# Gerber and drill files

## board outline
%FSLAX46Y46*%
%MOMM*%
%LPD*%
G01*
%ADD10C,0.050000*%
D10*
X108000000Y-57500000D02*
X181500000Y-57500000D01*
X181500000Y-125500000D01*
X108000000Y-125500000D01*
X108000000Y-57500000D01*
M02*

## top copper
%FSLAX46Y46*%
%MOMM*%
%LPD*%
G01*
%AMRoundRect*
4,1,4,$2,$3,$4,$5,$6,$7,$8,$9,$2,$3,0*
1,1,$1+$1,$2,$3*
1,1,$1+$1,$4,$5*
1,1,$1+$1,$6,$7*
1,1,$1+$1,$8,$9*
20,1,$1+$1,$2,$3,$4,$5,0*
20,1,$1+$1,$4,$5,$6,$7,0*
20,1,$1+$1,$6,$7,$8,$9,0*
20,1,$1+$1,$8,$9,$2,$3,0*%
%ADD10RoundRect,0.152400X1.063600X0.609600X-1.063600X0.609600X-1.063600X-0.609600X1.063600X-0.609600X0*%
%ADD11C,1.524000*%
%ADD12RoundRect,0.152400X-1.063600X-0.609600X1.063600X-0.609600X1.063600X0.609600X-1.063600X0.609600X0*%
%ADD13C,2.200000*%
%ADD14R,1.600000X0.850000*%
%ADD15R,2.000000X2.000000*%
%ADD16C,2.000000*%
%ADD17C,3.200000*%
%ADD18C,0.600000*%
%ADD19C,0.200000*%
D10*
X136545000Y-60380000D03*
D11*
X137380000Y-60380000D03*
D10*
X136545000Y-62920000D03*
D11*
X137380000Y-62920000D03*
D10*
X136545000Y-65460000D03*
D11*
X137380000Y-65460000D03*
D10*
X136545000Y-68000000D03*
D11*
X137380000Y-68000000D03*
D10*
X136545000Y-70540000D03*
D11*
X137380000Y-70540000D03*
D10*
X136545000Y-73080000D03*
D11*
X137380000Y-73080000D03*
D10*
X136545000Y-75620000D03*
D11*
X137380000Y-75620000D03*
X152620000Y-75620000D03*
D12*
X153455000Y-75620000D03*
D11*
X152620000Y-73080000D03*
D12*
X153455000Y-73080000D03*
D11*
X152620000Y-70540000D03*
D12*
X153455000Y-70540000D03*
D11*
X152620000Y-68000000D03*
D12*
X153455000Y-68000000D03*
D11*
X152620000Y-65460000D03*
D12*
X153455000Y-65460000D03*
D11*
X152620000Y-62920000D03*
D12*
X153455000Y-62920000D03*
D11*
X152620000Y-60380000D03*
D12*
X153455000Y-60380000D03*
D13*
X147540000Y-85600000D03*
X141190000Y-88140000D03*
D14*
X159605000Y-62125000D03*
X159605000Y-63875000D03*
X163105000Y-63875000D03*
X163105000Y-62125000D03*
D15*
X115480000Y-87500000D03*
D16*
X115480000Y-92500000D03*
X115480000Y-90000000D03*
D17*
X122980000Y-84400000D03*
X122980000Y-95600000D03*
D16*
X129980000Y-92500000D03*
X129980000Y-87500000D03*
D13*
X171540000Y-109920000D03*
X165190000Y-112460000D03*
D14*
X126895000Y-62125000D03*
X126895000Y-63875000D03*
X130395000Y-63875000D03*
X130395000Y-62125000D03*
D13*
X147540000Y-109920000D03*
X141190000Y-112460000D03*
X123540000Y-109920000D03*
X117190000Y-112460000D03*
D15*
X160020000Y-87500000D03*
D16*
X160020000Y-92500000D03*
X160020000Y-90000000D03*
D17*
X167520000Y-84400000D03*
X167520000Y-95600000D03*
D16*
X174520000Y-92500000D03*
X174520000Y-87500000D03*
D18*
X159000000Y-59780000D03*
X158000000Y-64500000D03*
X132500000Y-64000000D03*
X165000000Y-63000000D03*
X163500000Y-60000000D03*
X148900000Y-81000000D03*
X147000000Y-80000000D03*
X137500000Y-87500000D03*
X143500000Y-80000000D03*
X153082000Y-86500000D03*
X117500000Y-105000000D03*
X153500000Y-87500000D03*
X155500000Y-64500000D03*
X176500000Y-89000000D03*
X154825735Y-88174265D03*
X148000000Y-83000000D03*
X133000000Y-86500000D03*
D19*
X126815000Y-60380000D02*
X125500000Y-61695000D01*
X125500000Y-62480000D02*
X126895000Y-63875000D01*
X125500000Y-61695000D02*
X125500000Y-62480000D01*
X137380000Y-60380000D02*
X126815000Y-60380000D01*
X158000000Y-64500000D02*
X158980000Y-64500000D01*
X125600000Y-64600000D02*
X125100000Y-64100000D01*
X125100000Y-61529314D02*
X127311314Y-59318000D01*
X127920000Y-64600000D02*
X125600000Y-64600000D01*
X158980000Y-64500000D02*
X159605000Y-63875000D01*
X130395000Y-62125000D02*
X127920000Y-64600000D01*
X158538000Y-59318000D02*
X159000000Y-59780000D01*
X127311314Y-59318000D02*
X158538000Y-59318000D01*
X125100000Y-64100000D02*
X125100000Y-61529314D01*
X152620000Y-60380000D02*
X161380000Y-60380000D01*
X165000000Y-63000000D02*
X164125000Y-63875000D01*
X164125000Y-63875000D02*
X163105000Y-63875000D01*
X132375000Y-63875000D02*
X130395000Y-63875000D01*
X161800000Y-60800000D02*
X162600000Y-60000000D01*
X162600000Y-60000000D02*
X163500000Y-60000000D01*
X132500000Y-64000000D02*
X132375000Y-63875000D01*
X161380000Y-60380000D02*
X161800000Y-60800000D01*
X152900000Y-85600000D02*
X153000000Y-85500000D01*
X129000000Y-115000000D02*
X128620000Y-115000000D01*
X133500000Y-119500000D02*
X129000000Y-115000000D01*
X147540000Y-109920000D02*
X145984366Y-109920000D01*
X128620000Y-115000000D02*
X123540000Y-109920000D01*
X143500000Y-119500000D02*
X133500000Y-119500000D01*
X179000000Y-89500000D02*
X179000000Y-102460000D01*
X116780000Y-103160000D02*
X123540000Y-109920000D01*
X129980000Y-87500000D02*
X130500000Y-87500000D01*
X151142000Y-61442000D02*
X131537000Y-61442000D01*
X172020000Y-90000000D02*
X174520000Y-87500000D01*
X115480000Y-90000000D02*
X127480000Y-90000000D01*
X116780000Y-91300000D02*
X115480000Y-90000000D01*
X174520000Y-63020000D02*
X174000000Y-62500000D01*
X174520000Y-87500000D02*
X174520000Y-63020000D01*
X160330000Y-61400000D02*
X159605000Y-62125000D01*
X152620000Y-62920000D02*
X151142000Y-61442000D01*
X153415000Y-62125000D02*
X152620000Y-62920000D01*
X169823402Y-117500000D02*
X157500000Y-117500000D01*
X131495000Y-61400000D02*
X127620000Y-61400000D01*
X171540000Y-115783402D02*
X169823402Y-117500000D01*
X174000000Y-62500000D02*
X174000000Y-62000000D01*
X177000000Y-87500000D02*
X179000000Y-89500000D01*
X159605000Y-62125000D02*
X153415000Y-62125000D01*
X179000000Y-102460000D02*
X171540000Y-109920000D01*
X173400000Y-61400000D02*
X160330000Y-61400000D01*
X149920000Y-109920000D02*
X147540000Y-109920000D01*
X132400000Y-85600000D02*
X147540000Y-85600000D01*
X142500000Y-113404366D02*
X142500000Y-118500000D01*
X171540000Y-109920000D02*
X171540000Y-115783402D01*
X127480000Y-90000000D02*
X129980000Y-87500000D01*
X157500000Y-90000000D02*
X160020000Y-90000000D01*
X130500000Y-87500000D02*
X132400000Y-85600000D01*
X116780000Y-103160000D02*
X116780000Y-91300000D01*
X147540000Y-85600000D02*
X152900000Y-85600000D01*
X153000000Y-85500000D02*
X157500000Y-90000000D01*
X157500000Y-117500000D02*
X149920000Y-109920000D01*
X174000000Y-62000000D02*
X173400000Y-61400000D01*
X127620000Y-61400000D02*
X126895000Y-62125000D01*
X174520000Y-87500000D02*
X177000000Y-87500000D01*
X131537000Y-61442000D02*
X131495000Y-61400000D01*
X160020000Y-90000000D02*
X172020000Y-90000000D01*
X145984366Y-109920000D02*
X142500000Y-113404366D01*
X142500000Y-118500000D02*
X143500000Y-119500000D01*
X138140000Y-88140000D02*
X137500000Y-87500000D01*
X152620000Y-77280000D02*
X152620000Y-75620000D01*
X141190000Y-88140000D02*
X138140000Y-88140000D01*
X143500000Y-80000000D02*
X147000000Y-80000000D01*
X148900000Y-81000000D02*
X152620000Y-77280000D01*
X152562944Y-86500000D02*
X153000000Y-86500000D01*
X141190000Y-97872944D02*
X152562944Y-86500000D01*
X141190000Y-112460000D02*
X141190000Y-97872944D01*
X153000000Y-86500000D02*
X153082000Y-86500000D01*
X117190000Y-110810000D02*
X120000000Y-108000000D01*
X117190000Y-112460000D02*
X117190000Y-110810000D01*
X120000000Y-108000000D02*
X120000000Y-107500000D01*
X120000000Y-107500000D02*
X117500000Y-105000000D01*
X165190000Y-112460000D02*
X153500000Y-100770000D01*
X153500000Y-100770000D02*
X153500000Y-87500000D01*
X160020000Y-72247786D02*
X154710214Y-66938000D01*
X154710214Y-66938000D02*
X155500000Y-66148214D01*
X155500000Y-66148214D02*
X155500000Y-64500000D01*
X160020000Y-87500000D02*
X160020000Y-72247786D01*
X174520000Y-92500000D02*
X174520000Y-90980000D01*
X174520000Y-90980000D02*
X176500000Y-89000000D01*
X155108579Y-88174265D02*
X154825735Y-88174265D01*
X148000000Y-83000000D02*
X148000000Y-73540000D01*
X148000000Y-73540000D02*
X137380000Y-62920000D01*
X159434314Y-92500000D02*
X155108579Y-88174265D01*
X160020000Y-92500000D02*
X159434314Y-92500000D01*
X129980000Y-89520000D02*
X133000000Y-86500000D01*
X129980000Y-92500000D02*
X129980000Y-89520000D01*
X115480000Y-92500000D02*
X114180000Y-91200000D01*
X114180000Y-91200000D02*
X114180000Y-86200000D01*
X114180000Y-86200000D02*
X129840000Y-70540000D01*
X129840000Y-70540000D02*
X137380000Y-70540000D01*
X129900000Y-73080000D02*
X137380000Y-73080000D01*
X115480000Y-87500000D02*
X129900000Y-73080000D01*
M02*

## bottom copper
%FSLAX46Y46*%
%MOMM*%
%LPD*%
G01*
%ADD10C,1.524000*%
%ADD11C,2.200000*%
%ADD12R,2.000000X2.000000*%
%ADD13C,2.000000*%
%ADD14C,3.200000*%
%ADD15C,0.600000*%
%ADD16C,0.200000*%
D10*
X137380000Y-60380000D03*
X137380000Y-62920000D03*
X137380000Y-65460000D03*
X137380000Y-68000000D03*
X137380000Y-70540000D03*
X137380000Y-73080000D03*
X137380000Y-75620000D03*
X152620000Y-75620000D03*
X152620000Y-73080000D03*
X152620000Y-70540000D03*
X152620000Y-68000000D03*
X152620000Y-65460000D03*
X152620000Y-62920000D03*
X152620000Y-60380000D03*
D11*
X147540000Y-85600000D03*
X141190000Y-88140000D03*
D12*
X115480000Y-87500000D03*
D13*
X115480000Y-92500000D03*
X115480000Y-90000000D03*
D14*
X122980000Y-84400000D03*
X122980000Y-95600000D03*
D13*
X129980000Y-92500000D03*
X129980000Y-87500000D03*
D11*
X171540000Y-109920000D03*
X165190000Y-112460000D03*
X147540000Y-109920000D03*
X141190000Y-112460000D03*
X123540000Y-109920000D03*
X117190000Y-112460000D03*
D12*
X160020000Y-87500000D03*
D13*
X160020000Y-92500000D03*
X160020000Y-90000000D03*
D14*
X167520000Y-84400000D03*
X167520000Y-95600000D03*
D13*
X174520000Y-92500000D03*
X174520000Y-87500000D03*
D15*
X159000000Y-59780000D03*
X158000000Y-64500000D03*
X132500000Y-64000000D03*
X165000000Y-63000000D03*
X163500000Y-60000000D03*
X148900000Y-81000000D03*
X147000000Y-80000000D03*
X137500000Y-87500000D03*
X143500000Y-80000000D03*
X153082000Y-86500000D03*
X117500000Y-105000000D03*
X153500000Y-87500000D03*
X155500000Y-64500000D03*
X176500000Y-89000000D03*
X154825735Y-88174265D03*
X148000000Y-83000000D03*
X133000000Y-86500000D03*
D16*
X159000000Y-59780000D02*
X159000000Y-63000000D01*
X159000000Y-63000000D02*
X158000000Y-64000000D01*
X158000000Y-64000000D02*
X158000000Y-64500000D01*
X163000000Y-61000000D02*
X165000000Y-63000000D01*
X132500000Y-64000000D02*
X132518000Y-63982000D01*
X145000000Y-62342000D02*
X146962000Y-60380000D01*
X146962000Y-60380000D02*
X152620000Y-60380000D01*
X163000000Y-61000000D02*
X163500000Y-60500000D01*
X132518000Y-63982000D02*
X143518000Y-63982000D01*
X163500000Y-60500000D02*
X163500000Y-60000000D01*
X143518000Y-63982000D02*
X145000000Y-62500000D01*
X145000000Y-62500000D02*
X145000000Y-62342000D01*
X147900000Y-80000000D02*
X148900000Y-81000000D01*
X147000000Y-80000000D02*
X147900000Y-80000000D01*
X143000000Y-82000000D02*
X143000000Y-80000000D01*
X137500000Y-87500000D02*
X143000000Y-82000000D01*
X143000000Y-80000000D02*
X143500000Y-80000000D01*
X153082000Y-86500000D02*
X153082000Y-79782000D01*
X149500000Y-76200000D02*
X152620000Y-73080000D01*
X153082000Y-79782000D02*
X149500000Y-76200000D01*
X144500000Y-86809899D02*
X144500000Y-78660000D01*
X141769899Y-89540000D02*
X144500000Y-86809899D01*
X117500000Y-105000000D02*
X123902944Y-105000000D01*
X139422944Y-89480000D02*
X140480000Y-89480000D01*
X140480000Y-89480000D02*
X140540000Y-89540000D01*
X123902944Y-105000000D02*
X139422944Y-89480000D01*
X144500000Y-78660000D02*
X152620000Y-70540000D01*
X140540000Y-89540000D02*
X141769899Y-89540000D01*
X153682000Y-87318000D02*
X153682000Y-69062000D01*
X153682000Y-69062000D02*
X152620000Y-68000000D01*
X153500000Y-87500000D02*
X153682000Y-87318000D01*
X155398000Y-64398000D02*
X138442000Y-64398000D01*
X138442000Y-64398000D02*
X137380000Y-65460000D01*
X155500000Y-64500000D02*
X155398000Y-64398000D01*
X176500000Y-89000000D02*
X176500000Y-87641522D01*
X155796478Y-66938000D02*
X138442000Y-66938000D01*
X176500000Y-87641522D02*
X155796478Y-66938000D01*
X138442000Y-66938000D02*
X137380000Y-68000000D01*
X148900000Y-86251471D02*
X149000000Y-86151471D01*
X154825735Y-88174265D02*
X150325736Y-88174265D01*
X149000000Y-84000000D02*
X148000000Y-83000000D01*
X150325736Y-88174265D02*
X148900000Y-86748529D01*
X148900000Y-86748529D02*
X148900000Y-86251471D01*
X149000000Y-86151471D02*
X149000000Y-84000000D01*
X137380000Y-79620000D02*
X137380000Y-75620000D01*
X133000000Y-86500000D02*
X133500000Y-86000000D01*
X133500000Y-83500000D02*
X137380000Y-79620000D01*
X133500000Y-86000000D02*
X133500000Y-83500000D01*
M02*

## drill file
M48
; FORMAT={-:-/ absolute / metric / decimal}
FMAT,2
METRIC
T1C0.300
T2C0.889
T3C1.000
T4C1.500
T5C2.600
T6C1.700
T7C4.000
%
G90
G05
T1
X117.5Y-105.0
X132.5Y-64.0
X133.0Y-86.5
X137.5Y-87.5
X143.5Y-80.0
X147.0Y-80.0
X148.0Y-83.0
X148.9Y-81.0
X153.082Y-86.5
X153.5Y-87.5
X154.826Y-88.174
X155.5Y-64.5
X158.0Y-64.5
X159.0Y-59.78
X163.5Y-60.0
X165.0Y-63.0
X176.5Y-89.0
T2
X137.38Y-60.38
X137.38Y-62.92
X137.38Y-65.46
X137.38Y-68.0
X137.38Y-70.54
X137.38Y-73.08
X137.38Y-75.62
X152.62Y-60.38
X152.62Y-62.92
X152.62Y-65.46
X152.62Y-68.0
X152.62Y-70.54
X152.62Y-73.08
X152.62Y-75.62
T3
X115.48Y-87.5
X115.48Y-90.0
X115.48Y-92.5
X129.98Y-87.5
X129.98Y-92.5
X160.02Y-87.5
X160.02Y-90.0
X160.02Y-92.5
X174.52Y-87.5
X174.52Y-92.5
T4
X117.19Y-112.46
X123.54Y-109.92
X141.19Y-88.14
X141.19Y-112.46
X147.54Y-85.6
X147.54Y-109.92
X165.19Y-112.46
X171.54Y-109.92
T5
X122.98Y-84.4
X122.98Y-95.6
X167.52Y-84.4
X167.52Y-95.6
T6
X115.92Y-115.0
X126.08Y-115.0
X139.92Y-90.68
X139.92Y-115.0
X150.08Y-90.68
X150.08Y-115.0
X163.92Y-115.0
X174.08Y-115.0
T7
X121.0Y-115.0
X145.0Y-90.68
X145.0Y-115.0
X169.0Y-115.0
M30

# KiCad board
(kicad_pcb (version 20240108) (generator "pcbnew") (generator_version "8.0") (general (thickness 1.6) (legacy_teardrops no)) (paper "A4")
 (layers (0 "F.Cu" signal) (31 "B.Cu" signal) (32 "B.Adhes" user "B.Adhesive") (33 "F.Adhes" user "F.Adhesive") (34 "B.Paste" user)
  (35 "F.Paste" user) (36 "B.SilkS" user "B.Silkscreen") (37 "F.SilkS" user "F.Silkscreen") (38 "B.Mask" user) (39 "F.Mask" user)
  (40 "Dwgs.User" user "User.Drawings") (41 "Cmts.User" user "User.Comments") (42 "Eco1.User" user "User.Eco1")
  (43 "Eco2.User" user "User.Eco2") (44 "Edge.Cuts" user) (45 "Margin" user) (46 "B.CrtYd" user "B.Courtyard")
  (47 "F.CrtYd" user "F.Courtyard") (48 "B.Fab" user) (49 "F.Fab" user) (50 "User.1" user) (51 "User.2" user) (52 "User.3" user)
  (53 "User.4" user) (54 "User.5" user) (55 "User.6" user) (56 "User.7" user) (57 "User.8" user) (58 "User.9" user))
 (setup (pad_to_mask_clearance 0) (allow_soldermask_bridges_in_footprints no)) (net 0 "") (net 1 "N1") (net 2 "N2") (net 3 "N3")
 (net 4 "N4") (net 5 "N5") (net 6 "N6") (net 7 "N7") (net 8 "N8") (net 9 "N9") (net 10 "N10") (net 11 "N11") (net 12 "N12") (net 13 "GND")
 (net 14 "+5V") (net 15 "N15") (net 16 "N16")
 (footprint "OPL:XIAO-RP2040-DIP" (layer "F.Cu") (at 145 68)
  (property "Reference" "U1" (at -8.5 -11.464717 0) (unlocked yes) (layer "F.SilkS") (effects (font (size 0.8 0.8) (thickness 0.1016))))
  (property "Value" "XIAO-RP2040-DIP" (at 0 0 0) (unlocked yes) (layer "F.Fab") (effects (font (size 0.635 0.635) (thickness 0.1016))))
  (pad "1" smd roundrect (at -8.455 -7.62 180) (size 2.432 1.524) (layers "F.Cu" "F.Mask") (roundrect_rratio 0.1) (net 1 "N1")
   (thermal_bridge_angle 45))
  (pad "1" thru_hole circle (at -7.62 -7.62 180) (size 1.524 1.524) (drill 0.889) (layers "*.Cu" "*.Mask") (remove_unused_layers no)
   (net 1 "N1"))
  (pad "2" smd roundrect (at -8.455 -5.08 180) (size 2.432 1.524) (layers "F.Cu" "F.Mask") (roundrect_rratio 0.1) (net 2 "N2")
   (thermal_bridge_angle 45))
  (pad "2" thru_hole circle (at -7.62 -5.08 180) (size 1.524 1.524) (drill 0.889) (layers "*.Cu" "*.Mask") (remove_unused_layers no)
   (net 2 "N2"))
  (pad "3" smd roundrect (at -8.455 -2.54 180) (size 2.432 1.524) (layers "F.Cu" "F.Mask") (roundrect_rratio 0.1) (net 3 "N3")
   (thermal_bridge_angle 45))
  (pad "3" thru_hole circle (at -7.62 -2.54 180) (size 1.524 1.524) (drill 0.889) (layers "*.Cu" "*.Mask") (remove_unused_layers no)
   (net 3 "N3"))
  (pad "4" smd roundrect (at -8.455 0 180) (size 2.432 1.524) (layers "F.Cu" "F.Mask") (roundrect_rratio 0.1) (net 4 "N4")
   (thermal_bridge_angle 45))
  (pad "4" thru_hole circle (at -7.62 0 180) (size 1.524 1.524) (drill 0.889) (layers "*.Cu" "*.Mask") (remove_unused_layers no)
   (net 4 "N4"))
  (pad "5" smd roundrect (at -8.455 2.54 180) (size 2.432 1.524) (layers "F.Cu" "F.Mask") (roundrect_rratio 0.1) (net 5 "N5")
   (thermal_bridge_angle 45))
  (pad "5" thru_hole circle (at -7.62 2.54 180) (size 1.524 1.524) (drill 0.889) (layers "*.Cu" "*.Mask") (remove_unused_layers no)
   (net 5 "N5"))
  (pad "6" smd roundrect (at -8.455 5.08 180) (size 2.432 1.524) (layers "F.Cu" "F.Mask") (roundrect_rratio 0.1) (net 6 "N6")
   (thermal_bridge_angle 45))
  (pad "6" thru_hole circle (at -7.62 5.08 180) (size 1.524 1.524) (drill 0.889) (layers "*.Cu" "*.Mask") (remove_unused_layers no)
   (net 6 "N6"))
  (pad "7" smd roundrect (at -8.455 7.62 180) (size 2.432 1.524) (layers "F.Cu" "F.Mask") (roundrect_rratio 0.1) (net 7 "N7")
   (thermal_bridge_angle 45))
  (pad "7" thru_hole circle (at -7.62 7.62 180) (size 1.524 1.524) (drill 0.889) (layers "*.Cu" "*.Mask") (remove_unused_layers no)
   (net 7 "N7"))
  (pad "8" thru_hole circle (at 7.62 7.62) (size 1.524 1.524) (drill 0.889) (layers "*.Cu" "*.Mask") (remove_unused_layers no) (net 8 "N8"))
  (pad "8" smd roundrect (at 8.455 7.62) (size 2.432 1.524) (layers "F.Cu" "F.Mask") (roundrect_rratio 0.1) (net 8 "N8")
   (thermal_bridge_angle 45))
  (pad "9" thru_hole circle (at 7.62 5.08) (size 1.524 1.524) (drill 0.889) (layers "*.Cu" "*.Mask") (remove_unused_layers no) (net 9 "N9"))
  (pad "9" smd roundrect (at 8.455 5.08) (size 2.432 1.524) (layers "F.Cu" "F.Mask") (roundrect_rratio 0.1) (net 9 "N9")
   (thermal_bridge_angle 45))
  (pad "10" thru_hole circle (at 7.62 2.54) (size 1.524 1.524) (drill 0.889) (layers "*.Cu" "*.Mask") (remove_unused_layers no)
   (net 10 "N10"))
  (pad "10" smd roundrect (at 8.455 2.54) (size 2.432 1.524) (layers "F.Cu" "F.Mask") (roundrect_rratio 0.1) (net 10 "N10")
   (thermal_bridge_angle 45))
  (pad "11" thru_hole circle (at 7.62 0) (size 1.524 1.524) (drill 0.889) (layers "*.Cu" "*.Mask") (remove_unused_layers no) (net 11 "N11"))
  (pad "11" smd roundrect (at 8.455 0) (size 2.432 1.524) (layers "F.Cu" "F.Mask") (roundrect_rratio 0.1) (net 11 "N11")
   (thermal_bridge_angle 45))
  (pad "12" thru_hole circle (at 7.62 -2.54) (size 1.524 1.524) (drill 0.889) (layers "*.Cu" "*.Mask") (remove_unused_layers no)
   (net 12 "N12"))
  (pad "12" smd roundrect (at 8.455 -2.54) (size 2.432 1.524) (layers "F.Cu" "F.Mask") (roundrect_rratio 0.1) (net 12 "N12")
   (thermal_bridge_angle 45))
  (pad "13" thru_hole circle (at 7.62 -5.08) (size 1.524 1.524) (drill 0.889) (layers "*.Cu" "*.Mask") (remove_unused_layers no)
   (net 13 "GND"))
  (pad "13" smd roundrect (at 8.455 -5.08) (size 2.432 1.524) (layers "F.Cu" "F.Mask") (roundrect_rratio 0.1) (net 13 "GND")
   (thermal_bridge_angle 45))
  (pad "14" thru_hole circle (at 7.62 -7.62) (size 1.524 1.524) (drill 0.889) (layers "*.Cu" "*.Mask") (remove_unused_layers no)
   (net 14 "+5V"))
  (pad "14" smd roundrect (at 8.455 -7.62) (size 2.432 1.524) (layers "F.Cu" "F.Mask") (roundrect_rratio 0.1) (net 14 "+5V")
   (thermal_bridge_angle 45)))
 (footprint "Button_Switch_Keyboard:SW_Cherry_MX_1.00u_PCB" (layer "F.Cu") (at 147.54 85.6)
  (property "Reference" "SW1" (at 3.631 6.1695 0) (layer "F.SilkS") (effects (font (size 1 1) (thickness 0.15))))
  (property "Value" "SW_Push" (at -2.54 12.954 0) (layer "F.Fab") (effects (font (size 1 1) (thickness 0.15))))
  (pad "" np_thru_hole circle (at -7.62 5.08) (size 1.7 1.7) (drill 1.7) (layers "*.Cu" "*.Mask"))
  (pad "" np_thru_hole circle (at -2.54 5.08) (size 4 4) (drill 4) (layers "*.Cu" "*.Mask"))
  (pad "" np_thru_hole circle (at 2.54 5.08) (size 1.7 1.7) (drill 1.7) (layers "*.Cu" "*.Mask"))
  (pad "1" thru_hole circle (at 0 0) (size 2.2 2.2) (drill 1.5) (layers "*.Cu" "*.Mask") (remove_unused_layers no) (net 13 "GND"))
  (pad "2" thru_hole circle (at -6.35 2.54) (size 2.2 2.2) (drill 1.5) (layers "*.Cu" "*.Mask") (remove_unused_layers no) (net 8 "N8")))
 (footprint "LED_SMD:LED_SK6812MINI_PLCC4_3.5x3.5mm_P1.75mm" (layer "F.Cu") (at 161.355 63)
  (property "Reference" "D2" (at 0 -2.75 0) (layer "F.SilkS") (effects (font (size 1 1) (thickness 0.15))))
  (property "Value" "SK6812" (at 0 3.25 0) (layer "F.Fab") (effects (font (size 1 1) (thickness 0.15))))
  (pad "1" smd rect (at -1.75 -0.875) (size 1.6 0.85) (layers "F.Cu" "F.Paste" "F.Mask") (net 13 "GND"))
  (pad "2" smd rect (at -1.75 0.875) (size 1.6 0.85) (layers "F.Cu" "F.Paste" "F.Mask") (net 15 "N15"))
  (pad "3" smd rect (at 1.75 0.875) (size 1.6 0.85) (layers "F.Cu" "F.Paste" "F.Mask") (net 14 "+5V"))
  (pad "4" smd rect (at 1.75 -0.875) (size 1.6 0.85) (layers "F.Cu" "F.Paste" "F.Mask") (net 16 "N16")))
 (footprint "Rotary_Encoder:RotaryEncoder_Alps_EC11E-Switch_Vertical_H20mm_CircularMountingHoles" (layer "F.Cu") (at 115.48 87.5)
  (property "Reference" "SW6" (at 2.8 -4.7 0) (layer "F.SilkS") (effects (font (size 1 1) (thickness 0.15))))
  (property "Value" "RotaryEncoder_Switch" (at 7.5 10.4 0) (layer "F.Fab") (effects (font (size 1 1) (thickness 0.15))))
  (pad "A" thru_hole rect (at 0 0) (size 2 2) (drill 1) (layers "*.Cu" "*.Mask") (remove_unused_layers no) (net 6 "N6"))
  (pad "B" thru_hole circle (at 0 5) (size 2 2) (drill 1) (layers "*.Cu" "*.Mask") (remove_unused_layers no) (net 5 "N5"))
  (pad "C" thru_hole circle (at 0 2.5) (size 2 2) (drill 1) (layers "*.Cu" "*.Mask") (remove_unused_layers no) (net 13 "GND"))
  (pad "MP" thru_hole circle (at 7.5 -3.1) (size 3.2 3.2) (drill 2.6) (layers "*.Cu" "*.Mask") (remove_unused_layers no))
  (pad "MP" thru_hole circle (at 7.5 8.1) (size 3.2 3.2) (drill 2.6) (layers "*.Cu" "*.Mask") (remove_unused_layers no))
  (pad "S1" thru_hole circle (at 14.5 5) (size 2 2) (drill 1) (layers "*.Cu" "*.Mask") (remove_unused_layers no) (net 7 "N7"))
  (pad "S2" thru_hole circle (at 14.5 0) (size 2 2) (drill 1) (layers "*.Cu" "*.Mask") (remove_unused_layers no) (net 13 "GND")))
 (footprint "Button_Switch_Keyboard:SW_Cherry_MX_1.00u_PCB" (layer "F.Cu") (at 171.54 109.92)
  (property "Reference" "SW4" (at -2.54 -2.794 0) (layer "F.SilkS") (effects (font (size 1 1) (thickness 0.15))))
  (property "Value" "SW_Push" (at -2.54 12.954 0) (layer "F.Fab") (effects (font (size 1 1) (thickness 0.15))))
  (pad "" np_thru_hole circle (at -7.62 5.08) (size 1.7 1.7) (drill 1.7) (layers "*.Cu" "*.Mask"))
  (pad "" np_thru_hole circle (at -2.54 5.08) (size 4 4) (drill 4) (layers "*.Cu" "*.Mask"))
  (pad "" np_thru_hole circle (at 2.54 5.08) (size 1.7 1.7) (drill 1.7) (layers "*.Cu" "*.Mask"))
  (pad "1" thru_hole circle (at 0 0) (size 2.2 2.2) (drill 1.5) (layers "*.Cu" "*.Mask") (remove_unused_layers no) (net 13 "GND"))
  (pad "2" thru_hole circle (at -6.35 2.54) (size 2.2 2.2) (drill 1.5) (layers "*.Cu" "*.Mask") (remove_unused_layers no) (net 11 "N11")))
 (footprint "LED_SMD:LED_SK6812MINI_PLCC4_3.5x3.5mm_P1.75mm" (layer "F.Cu") (at 128.645 63)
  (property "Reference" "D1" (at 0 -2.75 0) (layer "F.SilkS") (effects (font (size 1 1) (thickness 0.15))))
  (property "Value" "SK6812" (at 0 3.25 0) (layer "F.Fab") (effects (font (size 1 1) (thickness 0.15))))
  (pad "1" smd rect (at -1.75 -0.875) (size 1.6 0.85) (layers "F.Cu" "F.Paste" "F.Mask") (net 13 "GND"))
  (pad "2" smd rect (at -1.75 0.875) (size 1.6 0.85) (layers "F.Cu" "F.Paste" "F.Mask") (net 1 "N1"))
  (pad "3" smd rect (at 1.75 0.875) (size 1.6 0.85) (layers "F.Cu" "F.Paste" "F.Mask") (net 14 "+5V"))
  (pad "4" smd rect (at 1.75 -0.875) (size 1.6 0.85) (layers "F.Cu" "F.Paste" "F.Mask") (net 15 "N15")))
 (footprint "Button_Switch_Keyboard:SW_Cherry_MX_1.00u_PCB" (layer "F.Cu") (at 147.54 109.92)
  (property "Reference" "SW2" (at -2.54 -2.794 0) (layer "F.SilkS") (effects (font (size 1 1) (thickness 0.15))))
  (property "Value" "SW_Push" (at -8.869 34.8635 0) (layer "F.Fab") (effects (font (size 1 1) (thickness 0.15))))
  (pad "" np_thru_hole circle (at -7.62 5.08) (size 1.7 1.7) (drill 1.7) (layers "*.Cu" "*.Mask"))
  (pad "" np_thru_hole circle (at -2.54 5.08) (size 4 4) (drill 4) (layers "*.Cu" "*.Mask"))
  (pad "" np_thru_hole circle (at 2.54 5.08) (size 1.7 1.7) (drill 1.7) (layers "*.Cu" "*.Mask"))
  (pad "1" thru_hole circle (at 0 0) (size 2.2 2.2) (drill 1.5) (layers "*.Cu" "*.Mask") (remove_unused_layers no) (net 13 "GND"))
  (pad "2" thru_hole circle (at -6.35 2.54) (size 2.2 2.2) (drill 1.5) (layers "*.Cu" "*.Mask") (remove_unused_layers no) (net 9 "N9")))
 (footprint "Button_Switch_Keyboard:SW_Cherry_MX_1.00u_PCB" (layer "F.Cu") (at 123.54 109.92)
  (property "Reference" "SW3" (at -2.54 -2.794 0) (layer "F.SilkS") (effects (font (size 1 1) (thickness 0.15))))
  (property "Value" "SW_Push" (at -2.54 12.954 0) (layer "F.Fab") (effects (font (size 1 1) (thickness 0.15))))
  (pad "" np_thru_hole circle (at -7.62 5.08) (size 1.7 1.7) (drill 1.7) (layers "*.Cu" "*.Mask"))
  (pad "" np_thru_hole circle (at -2.54 5.08) (size 4 4) (drill 4) (layers "*.Cu" "*.Mask"))
  (pad "" np_thru_hole circle (at 2.54 5.08) (size 1.7 1.7) (drill 1.7) (layers "*.Cu" "*.Mask"))
  (pad "1" thru_hole circle (at 0 0) (size 2.2 2.2) (drill 1.5) (layers "*.Cu" "*.Mask") (remove_unused_layers no) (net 13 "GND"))
  (pad "2" thru_hole circle (at -6.35 2.54) (size 2.2 2.2) (drill 1.5) (layers "*.Cu" "*.Mask") (remove_unused_layers no) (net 10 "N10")))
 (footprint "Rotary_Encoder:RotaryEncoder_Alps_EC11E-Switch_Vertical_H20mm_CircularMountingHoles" (layer "F.Cu") (at 160.02 87.5)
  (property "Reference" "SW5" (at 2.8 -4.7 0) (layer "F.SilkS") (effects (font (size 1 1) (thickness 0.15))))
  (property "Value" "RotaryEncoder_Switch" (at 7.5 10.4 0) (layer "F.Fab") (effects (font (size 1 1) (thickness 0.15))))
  (pad "A" thru_hole rect (at 0 0) (size 2 2) (drill 1) (layers "*.Cu" "*.Mask") (remove_unused_layers no) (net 3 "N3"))
  (pad "B" thru_hole circle (at 0 5) (size 2 2) (drill 1) (layers "*.Cu" "*.Mask") (remove_unused_layers no) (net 2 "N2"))
  (pad "C" thru_hole circle (at 0 2.5) (size 2 2) (drill 1) (layers "*.Cu" "*.Mask") (remove_unused_layers no) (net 13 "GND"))
  (pad "MP" thru_hole circle (at 7.5 -3.1) (size 3.2 3.2) (drill 2.6) (layers "*.Cu" "*.Mask") (remove_unused_layers no))
  (pad "MP" thru_hole circle (at 7.5 8.1) (size 3.2 3.2) (drill 2.6) (layers "*.Cu" "*.Mask") (remove_unused_layers no))
  (pad "S1" thru_hole circle (at 14.5 5) (size 2 2) (drill 1) (layers "*.Cu" "*.Mask") (remove_unused_layers no) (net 4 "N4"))
  (pad "S2" thru_hole circle (at 14.5 0) (size 2 2) (drill 1) (layers "*.Cu" "*.Mask") (remove_unused_layers no) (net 13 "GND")))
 (gr_rect (start 108 57.5) (end 181.5 125.5) (stroke (width 0.05) (type default)) (fill none) (layer "Edge.Cuts"))
 (segment (start 126.815 60.38) (end 125.5 61.695) (width 0.2) (layer "F.Cu") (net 1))
 (segment (start 125.5 62.48) (end 126.895 63.875) (width 0.2) (layer "F.Cu") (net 1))
 (segment (start 125.5 61.695) (end 125.5 62.48) (width 0.2) (layer "F.Cu") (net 1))
 (segment (start 137.38 60.38) (end 126.815 60.38) (width 0.2) (layer "F.Cu") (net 1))
 (segment (start 158 64.5) (end 158.98 64.5) (width 0.2) (layer "F.Cu") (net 15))
 (segment (start 125.6 64.6) (end 125.1 64.1) (width 0.2) (layer "F.Cu") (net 15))
 (segment (start 125.1 61.529314) (end 127.311314 59.318) (width 0.2) (layer "F.Cu") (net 15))
 (segment (start 127.92 64.6) (end 125.6 64.6) (width 0.2) (layer "F.Cu") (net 15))
 (segment (start 158.98 64.5) (end 159.605 63.875) (width 0.2) (layer "F.Cu") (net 15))
 (segment (start 130.395 62.125) (end 127.92 64.6) (width 0.2) (layer "F.Cu") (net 15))
 (segment (start 158.538 59.318) (end 159 59.78) (width 0.2) (layer "F.Cu") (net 15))
 (segment (start 127.311314 59.318) (end 158.538 59.318) (width 0.2) (layer "F.Cu") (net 15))
 (segment (start 125.1 64.1) (end 125.1 61.529314) (width 0.2) (layer "F.Cu") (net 15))
 (via (at 159 59.78) (size 0.6) (drill 0.3) (layers "F.Cu" "B.Cu") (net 15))
 (via (at 158 64.5) (size 0.6) (drill 0.3) (layers "F.Cu" "B.Cu") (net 15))
 (segment (start 159 59.78) (end 159 63) (width 0.2) (layer "B.Cu") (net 15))
 (segment (start 159 63) (end 158 64) (width 0.2) (layer "B.Cu") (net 15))
 (segment (start 158 64) (end 158 64.5) (width 0.2) (layer "B.Cu") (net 15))
 (segment (start 152.62 60.38) (end 161.38 60.38) (width 0.2) (layer "F.Cu") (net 14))
 (segment (start 165 63) (end 164.125 63.875) (width 0.2) (layer "F.Cu") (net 14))
 (segment (start 164.125 63.875) (end 163.105 63.875) (width 0.2) (layer "F.Cu") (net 14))
 (segment (start 132.375 63.875) (end 130.395 63.875) (width 0.2) (layer "F.Cu") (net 14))
 (segment (start 161.8 60.8) (end 162.6 60) (width 0.2) (layer "F.Cu") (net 14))
 (segment (start 162.6 60) (end 163.5 60) (width 0.2) (layer "F.Cu") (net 14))
 (segment (start 132.5 64) (end 132.375 63.875) (width 0.2) (layer "F.Cu") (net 14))
 (segment (start 161.38 60.38) (end 161.8 60.8) (width 0.2) (layer "F.Cu") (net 14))
 (via (at 132.5 64) (size 0.6) (drill 0.3) (layers "F.Cu" "B.Cu") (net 14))
 (via (at 165 63) (size 0.6) (drill 0.3) (layers "F.Cu" "B.Cu") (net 14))
 (via (at 163.5 60) (size 0.6) (drill 0.3) (layers "F.Cu" "B.Cu") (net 14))
 (segment (start 163 61) (end 165 63) (width 0.2) (layer "B.Cu") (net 14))
 (segment (start 132.5 64) (end 132.518 63.982) (width 0.2) (layer "B.Cu") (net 14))
 (segment (start 145 62.342) (end 146.962 60.38) (width 0.2) (layer "B.Cu") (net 14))
 (segment (start 146.962 60.38) (end 152.62 60.38) (width 0.2) (layer "B.Cu") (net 14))
 (segment (start 163 61) (end 163.5 60.5) (width 0.2) (layer "B.Cu") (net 14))
 (segment (start 132.518 63.982) (end 143.518 63.982) (width 0.2) (layer "B.Cu") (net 14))
 (segment (start 163.5 60.5) (end 163.5 60) (width 0.2) (layer "B.Cu") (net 14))
 (segment (start 143.518 63.982) (end 145 62.5) (width 0.2) (layer "B.Cu") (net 14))
 (segment (start 145 62.5) (end 145 62.342) (width 0.2) (layer "B.Cu") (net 14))
 (segment (start 152.9 85.6) (end 153 85.5) (width 0.2) (layer "F.Cu") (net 13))
 (segment (start 129 115) (end 128.62 115) (width 0.2) (layer "F.Cu") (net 13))
 (segment (start 133.5 119.5) (end 129 115) (width 0.2) (layer "F.Cu") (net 13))
 (segment (start 147.54 109.92) (end 145.984366 109.92) (width 0.2) (layer "F.Cu") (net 13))
 (segment (start 128.62 115) (end 123.54 109.92) (width 0.2) (layer "F.Cu") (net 13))
 (segment (start 143.5 119.5) (end 133.5 119.5) (width 0.2) (layer "F.Cu") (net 13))
 (segment (start 179 89.5) (end 179 102.46) (width 0.2) (layer "F.Cu") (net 13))
 (segment (start 116.78 103.16) (end 123.54 109.92) (width 0.2) (layer "F.Cu") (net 13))
 (segment (start 129.98 87.5) (end 130.5 87.5) (width 0.2) (layer "F.Cu") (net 13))
 (segment (start 151.142 61.442) (end 131.537 61.442) (width 0.2) (layer "F.Cu") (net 13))
 (segment (start 172.02 90) (end 174.52 87.5) (width 0.2) (layer "F.Cu") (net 13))
 (segment (start 115.48 90) (end 127.48 90) (width 0.2) (layer "F.Cu") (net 13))
 (segment (start 116.78 91.3) (end 115.48 90) (width 0.2) (layer "F.Cu") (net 13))
 (segment (start 174.52 63.02) (end 174 62.5) (width 0.2) (layer "F.Cu") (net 13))
 (segment (start 174.52 87.5) (end 174.52 63.02) (width 0.2) (layer "F.Cu") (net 13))
 (segment (start 160.33 61.4) (end 159.605 62.125) (width 0.2) (layer "F.Cu") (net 13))
 (segment (start 152.62 62.92) (end 151.142 61.442) (width 0.2) (layer "F.Cu") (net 13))
 (segment (start 153.415 62.125) (end 152.62 62.92) (width 0.2) (layer "F.Cu") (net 13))
 (segment (start 169.823402 117.5) (end 157.5 117.5) (width 0.2) (layer "F.Cu") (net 13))
 (segment (start 131.495 61.4) (end 127.62 61.4) (width 0.2) (layer "F.Cu") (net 13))
 (segment (start 171.54 115.783402) (end 169.823402 117.5) (width 0.2) (layer "F.Cu") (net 13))
 (segment (start 174 62.5) (end 174 62) (width 0.2) (layer "F.Cu") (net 13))
 (segment (start 177 87.5) (end 179 89.5) (width 0.2) (layer "F.Cu") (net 13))
 (segment (start 159.605 62.125) (end 153.415 62.125) (width 0.2) (layer "F.Cu") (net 13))
 (segment (start 179 102.46) (end 171.54 109.92) (width 0.2) (layer "F.Cu") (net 13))
 (segment (start 173.4 61.4) (end 160.33 61.4) (width 0.2) (layer "F.Cu") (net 13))
 (segment (start 149.92 109.92) (end 147.54 109.92) (width 0.2) (layer "F.Cu") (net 13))
 (segment (start 132.4 85.6) (end 147.54 85.6) (width 0.2) (layer "F.Cu") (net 13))
 (segment (start 142.5 113.404366) (end 142.5 118.5) (width 0.2) (layer "F.Cu") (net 13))
 (segment (start 171.54 109.92) (end 171.54 115.783402) (width 0.2) (layer "F.Cu") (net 13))
 (segment (start 127.48 90) (end 129.98 87.5) (width 0.2) (layer "F.Cu") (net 13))
 (segment (start 157.5 90) (end 160.02 90) (width 0.2) (layer "F.Cu") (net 13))
 (segment (start 130.5 87.5) (end 132.4 85.6) (width 0.2) (layer "F.Cu") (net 13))
 (segment (start 116.78 103.16) (end 116.78 91.3) (width 0.2) (layer "F.Cu") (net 13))
 (segment (start 147.54 85.6) (end 152.9 85.6) (width 0.2) (layer "F.Cu") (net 13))
 (segment (start 153 85.5) (end 157.5 90) (width 0.2) (layer "F.Cu") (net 13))
 (segment (start 157.5 117.5) (end 149.92 109.92) (width 0.2) (layer "F.Cu") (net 13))
 (segment (start 174 62) (end 173.4 61.4) (width 0.2) (layer "F.Cu") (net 13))
 (segment (start 127.62 61.4) (end 126.895 62.125) (width 0.2) (layer "F.Cu") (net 13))
 (segment (start 174.52 87.5) (end 177 87.5) (width 0.2) (layer "F.Cu") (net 13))
 (segment (start 131.537 61.442) (end 131.495 61.4) (width 0.2) (layer "F.Cu") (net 13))
 (segment (start 160.02 90) (end 172.02 90) (width 0.2) (layer "F.Cu") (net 13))
 (segment (start 145.984366 109.92) (end 142.5 113.404366) (width 0.2) (layer "F.Cu") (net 13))
 (segment (start 142.5 118.5) (end 143.5 119.5) (width 0.2) (layer "F.Cu") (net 13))
 (segment (start 138.14 88.14) (end 137.5 87.5) (width 0.2) (layer "F.Cu") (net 8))
 (segment (start 152.62 77.28) (end 152.62 75.62) (width 0.2) (layer "F.Cu") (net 8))
 (segment (start 141.19 88.14) (end 138.14 88.14) (width 0.2) (layer "F.Cu") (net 8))
 (segment (start 143.5 80) (end 147 80) (width 0.2) (layer "F.Cu") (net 8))
 (segment (start 148.9 81) (end 152.62 77.28) (width 0.2) (layer "F.Cu") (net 8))
 (via (at 148.9 81) (size 0.6) (drill 0.3) (layers "F.Cu" "B.Cu") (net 8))
 (via (at 147 80) (size 0.6) (drill 0.3) (layers "F.Cu" "B.Cu") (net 8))
 (via (at 137.5 87.5) (size 0.6) (drill 0.3) (layers "F.Cu" "B.Cu") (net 8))
 (via (at 143.5 80) (size 0.6) (drill 0.3) (layers "F.Cu" "B.Cu") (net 8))
 (segment (start 147.9 80) (end 148.9 81) (width 0.2) (layer "B.Cu") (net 8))
 (segment (start 147 80) (end 147.9 80) (width 0.2) (layer "B.Cu") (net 8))
 (segment (start 143 82) (end 143 80) (width 0.2) (layer "B.Cu") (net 8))
 (segment (start 137.5 87.5) (end 143 82) (width 0.2) (layer "B.Cu") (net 8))
 (segment (start 143 80) (end 143.5 80) (width 0.2) (layer "B.Cu") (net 8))
 (segment (start 152.562944 86.5) (end 153 86.5) (width 0.2) (layer "F.Cu") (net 9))
 (segment (start 141.19 97.872944) (end 152.562944 86.5) (width 0.2) (layer "F.Cu") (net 9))
 (segment (start 141.19 112.46) (end 141.19 97.872944) (width 0.2) (layer "F.Cu") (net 9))
 (segment (start 153 86.5) (end 153.082 86.5) (width 0.2) (layer "F.Cu") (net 9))
 (via (at 153.082 86.5) (size 0.6) (drill 0.3) (layers "F.Cu" "B.Cu") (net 9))
 (segment (start 153.082 86.5) (end 153.082 79.782) (width 0.2) (layer "B.Cu") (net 9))
 (segment (start 149.5 76.2) (end 152.62 73.08) (width 0.2) (layer "B.Cu") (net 9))
 (segment (start 153.082 79.782) (end 149.5 76.2) (width 0.2) (layer "B.Cu") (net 9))
 (segment (start 117.19 110.81) (end 120 108) (width 0.2) (layer "F.Cu") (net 10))
 (segment (start 117.19 112.46) (end 117.19 110.81) (width 0.2) (layer "F.Cu") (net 10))
 (segment (start 120 108) (end 120 107.5) (width 0.2) (layer "F.Cu") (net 10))
 (segment (start 120 107.5) (end 117.5 105) (width 0.2) (layer "F.Cu") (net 10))
 (via (at 117.5 105) (size 0.6) (drill 0.3) (layers "F.Cu" "B.Cu") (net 10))
 (segment (start 144.5 86.809899) (end 144.5 78.66) (width 0.2) (layer "B.Cu") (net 10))
 (segment (start 141.769899 89.54) (end 144.5 86.809899) (width 0.2) (layer "B.Cu") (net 10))
 (segment (start 117.5 105) (end 123.902944 105) (width 0.2) (layer "B.Cu") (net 10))
 (segment (start 139.422944 89.48) (end 140.48 89.48) (width 0.2) (layer "B.Cu") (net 10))
 (segment (start 140.48 89.48) (end 140.54 89.54) (width 0.2) (layer "B.Cu") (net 10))
 (segment (start 123.902944 105) (end 139.422944 89.48) (width 0.2) (layer "B.Cu") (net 10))
 (segment (start 144.5 78.66) (end 152.62 70.54) (width 0.2) (layer "B.Cu") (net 10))
 (segment (start 140.54 89.54) (end 141.769899 89.54) (width 0.2) (layer "B.Cu") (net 10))
 (segment (start 165.19 112.46) (end 153.5 100.77) (width 0.2) (layer "F.Cu") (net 11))
 (segment (start 153.5 100.77) (end 153.5 87.5) (width 0.2) (layer "F.Cu") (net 11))
 (via (at 153.5 87.5) (size 0.6) (drill 0.3) (layers "F.Cu" "B.Cu") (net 11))
 (segment (start 153.682 87.318) (end 153.682 69.062) (width 0.2) (layer "B.Cu") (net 11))
 (segment (start 153.682 69.062) (end 152.62 68) (width 0.2) (layer "B.Cu") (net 11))
 (segment (start 153.5 87.5) (end 153.682 87.318) (width 0.2) (layer "B.Cu") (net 11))
 (segment (start 160.02 72.247786) (end 154.710214 66.938) (width 0.2) (layer "F.Cu") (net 3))
 (segment (start 154.710214 66.938) (end 155.5 66.148214) (width 0.2) (layer "F.Cu") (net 3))
 (segment (start 155.5 66.148214) (end 155.5 64.5) (width 0.2) (layer "F.Cu") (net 3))
 (segment (start 160.02 87.5) (end 160.02 72.247786) (width 0.2) (layer "F.Cu") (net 3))
 (via (at 155.5 64.5) (size 0.6) (drill 0.3) (layers "F.Cu" "B.Cu") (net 3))
 (segment (start 155.398 64.398) (end 138.442 64.398) (width 0.2) (layer "B.Cu") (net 3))
 (segment (start 138.442 64.398) (end 137.38 65.46) (width 0.2) (layer "B.Cu") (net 3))
 (segment (start 155.5 64.5) (end 155.398 64.398) (width 0.2) (layer "B.Cu") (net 3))
 (segment (start 174.52 92.5) (end 174.52 90.98) (width 0.2) (layer "F.Cu") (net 4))
 (segment (start 174.52 90.98) (end 176.5 89) (width 0.2) (layer "F.Cu") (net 4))
 (via (at 176.5 89) (size 0.6) (drill 0.3) (layers "F.Cu" "B.Cu") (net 4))
 (segment (start 176.5 89) (end 176.5 87.641522) (width 0.2) (layer "B.Cu") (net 4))
 (segment (start 155.796478 66.938) (end 138.442 66.938) (width 0.2) (layer "B.Cu") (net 4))
 (segment (start 176.5 87.641522) (end 155.796478 66.938) (width 0.2) (layer "B.Cu") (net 4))
 (segment (start 138.442 66.938) (end 137.38 68) (width 0.2) (layer "B.Cu") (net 4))
 (segment (start 155.108579 88.174265) (end 154.825735 88.174265) (width 0.2) (layer "F.Cu") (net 2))
 (segment (start 148 83) (end 148 73.54) (width 0.2) (layer "F.Cu") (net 2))
 (segment (start 148 73.54) (end 137.38 62.92) (width 0.2) (layer "F.Cu") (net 2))
 (segment (start 159.434314 92.5) (end 155.108579 88.174265) (width 0.2) (layer "F.Cu") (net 2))
 (segment (start 160.02 92.5) (end 159.434314 92.5) (width 0.2) (layer "F.Cu") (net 2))
 (via (at 154.825735 88.174265) (size 0.6) (drill 0.3) (layers "F.Cu" "B.Cu") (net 2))
 (via (at 148 83) (size 0.6) (drill 0.3) (layers "F.Cu" "B.Cu") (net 2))
 (segment (start 148.9 86.251471) (end 149 86.151471) (width 0.2) (layer "B.Cu") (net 2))
 (segment (start 154.825735 88.174265) (end 150.325736 88.174265) (width 0.2) (layer "B.Cu") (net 2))
 (segment (start 149 84) (end 148 83) (width 0.2) (layer "B.Cu") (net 2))
 (segment (start 150.325736 88.174265) (end 148.9 86.748529) (width 0.2) (layer "B.Cu") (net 2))
 (segment (start 148.9 86.748529) (end 148.9 86.251471) (width 0.2) (layer "B.Cu") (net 2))
 (segment (start 149 86.151471) (end 149 84) (width 0.2) (layer "B.Cu") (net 2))
 (segment (start 129.98 89.52) (end 133 86.5) (width 0.2) (layer "F.Cu") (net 7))
 (segment (start 129.98 92.5) (end 129.98 89.52) (width 0.2) (layer "F.Cu") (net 7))
 (via (at 133 86.5) (size 0.6) (drill 0.3) (layers "F.Cu" "B.Cu") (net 7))
 (segment (start 137.38 79.62) (end 137.38 75.62) (width 0.2) (layer "B.Cu") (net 7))
 (segment (start 133 86.5) (end 133.5 86) (width 0.2) (layer "B.Cu") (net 7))
 (segment (start 133.5 83.5) (end 137.38 79.62) (width 0.2) (layer "B.Cu") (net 7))
 (segment (start 133.5 86) (end 133.5 83.5) (width 0.2) (layer "B.Cu") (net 7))
 (segment (start 115.48 92.5) (end 114.18 91.2) (width 0.2) (layer "F.Cu") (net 5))
 (segment (start 114.18 91.2) (end 114.18 86.2) (width 0.2) (layer "F.Cu") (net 5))
 (segment (start 114.18 86.2) (end 129.84 70.54) (width 0.2) (layer "F.Cu") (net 5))
 (segment (start 129.84 70.54) (end 137.38 70.54) (width 0.2) (layer "F.Cu") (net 5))
 (segment (start 129.9 73.08) (end 137.38 73.08) (width 0.2) (layer "F.Cu") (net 6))
 (segment (start 115.48 87.5) (end 129.9 73.08) (width 0.2) (layer "F.Cu") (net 6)))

